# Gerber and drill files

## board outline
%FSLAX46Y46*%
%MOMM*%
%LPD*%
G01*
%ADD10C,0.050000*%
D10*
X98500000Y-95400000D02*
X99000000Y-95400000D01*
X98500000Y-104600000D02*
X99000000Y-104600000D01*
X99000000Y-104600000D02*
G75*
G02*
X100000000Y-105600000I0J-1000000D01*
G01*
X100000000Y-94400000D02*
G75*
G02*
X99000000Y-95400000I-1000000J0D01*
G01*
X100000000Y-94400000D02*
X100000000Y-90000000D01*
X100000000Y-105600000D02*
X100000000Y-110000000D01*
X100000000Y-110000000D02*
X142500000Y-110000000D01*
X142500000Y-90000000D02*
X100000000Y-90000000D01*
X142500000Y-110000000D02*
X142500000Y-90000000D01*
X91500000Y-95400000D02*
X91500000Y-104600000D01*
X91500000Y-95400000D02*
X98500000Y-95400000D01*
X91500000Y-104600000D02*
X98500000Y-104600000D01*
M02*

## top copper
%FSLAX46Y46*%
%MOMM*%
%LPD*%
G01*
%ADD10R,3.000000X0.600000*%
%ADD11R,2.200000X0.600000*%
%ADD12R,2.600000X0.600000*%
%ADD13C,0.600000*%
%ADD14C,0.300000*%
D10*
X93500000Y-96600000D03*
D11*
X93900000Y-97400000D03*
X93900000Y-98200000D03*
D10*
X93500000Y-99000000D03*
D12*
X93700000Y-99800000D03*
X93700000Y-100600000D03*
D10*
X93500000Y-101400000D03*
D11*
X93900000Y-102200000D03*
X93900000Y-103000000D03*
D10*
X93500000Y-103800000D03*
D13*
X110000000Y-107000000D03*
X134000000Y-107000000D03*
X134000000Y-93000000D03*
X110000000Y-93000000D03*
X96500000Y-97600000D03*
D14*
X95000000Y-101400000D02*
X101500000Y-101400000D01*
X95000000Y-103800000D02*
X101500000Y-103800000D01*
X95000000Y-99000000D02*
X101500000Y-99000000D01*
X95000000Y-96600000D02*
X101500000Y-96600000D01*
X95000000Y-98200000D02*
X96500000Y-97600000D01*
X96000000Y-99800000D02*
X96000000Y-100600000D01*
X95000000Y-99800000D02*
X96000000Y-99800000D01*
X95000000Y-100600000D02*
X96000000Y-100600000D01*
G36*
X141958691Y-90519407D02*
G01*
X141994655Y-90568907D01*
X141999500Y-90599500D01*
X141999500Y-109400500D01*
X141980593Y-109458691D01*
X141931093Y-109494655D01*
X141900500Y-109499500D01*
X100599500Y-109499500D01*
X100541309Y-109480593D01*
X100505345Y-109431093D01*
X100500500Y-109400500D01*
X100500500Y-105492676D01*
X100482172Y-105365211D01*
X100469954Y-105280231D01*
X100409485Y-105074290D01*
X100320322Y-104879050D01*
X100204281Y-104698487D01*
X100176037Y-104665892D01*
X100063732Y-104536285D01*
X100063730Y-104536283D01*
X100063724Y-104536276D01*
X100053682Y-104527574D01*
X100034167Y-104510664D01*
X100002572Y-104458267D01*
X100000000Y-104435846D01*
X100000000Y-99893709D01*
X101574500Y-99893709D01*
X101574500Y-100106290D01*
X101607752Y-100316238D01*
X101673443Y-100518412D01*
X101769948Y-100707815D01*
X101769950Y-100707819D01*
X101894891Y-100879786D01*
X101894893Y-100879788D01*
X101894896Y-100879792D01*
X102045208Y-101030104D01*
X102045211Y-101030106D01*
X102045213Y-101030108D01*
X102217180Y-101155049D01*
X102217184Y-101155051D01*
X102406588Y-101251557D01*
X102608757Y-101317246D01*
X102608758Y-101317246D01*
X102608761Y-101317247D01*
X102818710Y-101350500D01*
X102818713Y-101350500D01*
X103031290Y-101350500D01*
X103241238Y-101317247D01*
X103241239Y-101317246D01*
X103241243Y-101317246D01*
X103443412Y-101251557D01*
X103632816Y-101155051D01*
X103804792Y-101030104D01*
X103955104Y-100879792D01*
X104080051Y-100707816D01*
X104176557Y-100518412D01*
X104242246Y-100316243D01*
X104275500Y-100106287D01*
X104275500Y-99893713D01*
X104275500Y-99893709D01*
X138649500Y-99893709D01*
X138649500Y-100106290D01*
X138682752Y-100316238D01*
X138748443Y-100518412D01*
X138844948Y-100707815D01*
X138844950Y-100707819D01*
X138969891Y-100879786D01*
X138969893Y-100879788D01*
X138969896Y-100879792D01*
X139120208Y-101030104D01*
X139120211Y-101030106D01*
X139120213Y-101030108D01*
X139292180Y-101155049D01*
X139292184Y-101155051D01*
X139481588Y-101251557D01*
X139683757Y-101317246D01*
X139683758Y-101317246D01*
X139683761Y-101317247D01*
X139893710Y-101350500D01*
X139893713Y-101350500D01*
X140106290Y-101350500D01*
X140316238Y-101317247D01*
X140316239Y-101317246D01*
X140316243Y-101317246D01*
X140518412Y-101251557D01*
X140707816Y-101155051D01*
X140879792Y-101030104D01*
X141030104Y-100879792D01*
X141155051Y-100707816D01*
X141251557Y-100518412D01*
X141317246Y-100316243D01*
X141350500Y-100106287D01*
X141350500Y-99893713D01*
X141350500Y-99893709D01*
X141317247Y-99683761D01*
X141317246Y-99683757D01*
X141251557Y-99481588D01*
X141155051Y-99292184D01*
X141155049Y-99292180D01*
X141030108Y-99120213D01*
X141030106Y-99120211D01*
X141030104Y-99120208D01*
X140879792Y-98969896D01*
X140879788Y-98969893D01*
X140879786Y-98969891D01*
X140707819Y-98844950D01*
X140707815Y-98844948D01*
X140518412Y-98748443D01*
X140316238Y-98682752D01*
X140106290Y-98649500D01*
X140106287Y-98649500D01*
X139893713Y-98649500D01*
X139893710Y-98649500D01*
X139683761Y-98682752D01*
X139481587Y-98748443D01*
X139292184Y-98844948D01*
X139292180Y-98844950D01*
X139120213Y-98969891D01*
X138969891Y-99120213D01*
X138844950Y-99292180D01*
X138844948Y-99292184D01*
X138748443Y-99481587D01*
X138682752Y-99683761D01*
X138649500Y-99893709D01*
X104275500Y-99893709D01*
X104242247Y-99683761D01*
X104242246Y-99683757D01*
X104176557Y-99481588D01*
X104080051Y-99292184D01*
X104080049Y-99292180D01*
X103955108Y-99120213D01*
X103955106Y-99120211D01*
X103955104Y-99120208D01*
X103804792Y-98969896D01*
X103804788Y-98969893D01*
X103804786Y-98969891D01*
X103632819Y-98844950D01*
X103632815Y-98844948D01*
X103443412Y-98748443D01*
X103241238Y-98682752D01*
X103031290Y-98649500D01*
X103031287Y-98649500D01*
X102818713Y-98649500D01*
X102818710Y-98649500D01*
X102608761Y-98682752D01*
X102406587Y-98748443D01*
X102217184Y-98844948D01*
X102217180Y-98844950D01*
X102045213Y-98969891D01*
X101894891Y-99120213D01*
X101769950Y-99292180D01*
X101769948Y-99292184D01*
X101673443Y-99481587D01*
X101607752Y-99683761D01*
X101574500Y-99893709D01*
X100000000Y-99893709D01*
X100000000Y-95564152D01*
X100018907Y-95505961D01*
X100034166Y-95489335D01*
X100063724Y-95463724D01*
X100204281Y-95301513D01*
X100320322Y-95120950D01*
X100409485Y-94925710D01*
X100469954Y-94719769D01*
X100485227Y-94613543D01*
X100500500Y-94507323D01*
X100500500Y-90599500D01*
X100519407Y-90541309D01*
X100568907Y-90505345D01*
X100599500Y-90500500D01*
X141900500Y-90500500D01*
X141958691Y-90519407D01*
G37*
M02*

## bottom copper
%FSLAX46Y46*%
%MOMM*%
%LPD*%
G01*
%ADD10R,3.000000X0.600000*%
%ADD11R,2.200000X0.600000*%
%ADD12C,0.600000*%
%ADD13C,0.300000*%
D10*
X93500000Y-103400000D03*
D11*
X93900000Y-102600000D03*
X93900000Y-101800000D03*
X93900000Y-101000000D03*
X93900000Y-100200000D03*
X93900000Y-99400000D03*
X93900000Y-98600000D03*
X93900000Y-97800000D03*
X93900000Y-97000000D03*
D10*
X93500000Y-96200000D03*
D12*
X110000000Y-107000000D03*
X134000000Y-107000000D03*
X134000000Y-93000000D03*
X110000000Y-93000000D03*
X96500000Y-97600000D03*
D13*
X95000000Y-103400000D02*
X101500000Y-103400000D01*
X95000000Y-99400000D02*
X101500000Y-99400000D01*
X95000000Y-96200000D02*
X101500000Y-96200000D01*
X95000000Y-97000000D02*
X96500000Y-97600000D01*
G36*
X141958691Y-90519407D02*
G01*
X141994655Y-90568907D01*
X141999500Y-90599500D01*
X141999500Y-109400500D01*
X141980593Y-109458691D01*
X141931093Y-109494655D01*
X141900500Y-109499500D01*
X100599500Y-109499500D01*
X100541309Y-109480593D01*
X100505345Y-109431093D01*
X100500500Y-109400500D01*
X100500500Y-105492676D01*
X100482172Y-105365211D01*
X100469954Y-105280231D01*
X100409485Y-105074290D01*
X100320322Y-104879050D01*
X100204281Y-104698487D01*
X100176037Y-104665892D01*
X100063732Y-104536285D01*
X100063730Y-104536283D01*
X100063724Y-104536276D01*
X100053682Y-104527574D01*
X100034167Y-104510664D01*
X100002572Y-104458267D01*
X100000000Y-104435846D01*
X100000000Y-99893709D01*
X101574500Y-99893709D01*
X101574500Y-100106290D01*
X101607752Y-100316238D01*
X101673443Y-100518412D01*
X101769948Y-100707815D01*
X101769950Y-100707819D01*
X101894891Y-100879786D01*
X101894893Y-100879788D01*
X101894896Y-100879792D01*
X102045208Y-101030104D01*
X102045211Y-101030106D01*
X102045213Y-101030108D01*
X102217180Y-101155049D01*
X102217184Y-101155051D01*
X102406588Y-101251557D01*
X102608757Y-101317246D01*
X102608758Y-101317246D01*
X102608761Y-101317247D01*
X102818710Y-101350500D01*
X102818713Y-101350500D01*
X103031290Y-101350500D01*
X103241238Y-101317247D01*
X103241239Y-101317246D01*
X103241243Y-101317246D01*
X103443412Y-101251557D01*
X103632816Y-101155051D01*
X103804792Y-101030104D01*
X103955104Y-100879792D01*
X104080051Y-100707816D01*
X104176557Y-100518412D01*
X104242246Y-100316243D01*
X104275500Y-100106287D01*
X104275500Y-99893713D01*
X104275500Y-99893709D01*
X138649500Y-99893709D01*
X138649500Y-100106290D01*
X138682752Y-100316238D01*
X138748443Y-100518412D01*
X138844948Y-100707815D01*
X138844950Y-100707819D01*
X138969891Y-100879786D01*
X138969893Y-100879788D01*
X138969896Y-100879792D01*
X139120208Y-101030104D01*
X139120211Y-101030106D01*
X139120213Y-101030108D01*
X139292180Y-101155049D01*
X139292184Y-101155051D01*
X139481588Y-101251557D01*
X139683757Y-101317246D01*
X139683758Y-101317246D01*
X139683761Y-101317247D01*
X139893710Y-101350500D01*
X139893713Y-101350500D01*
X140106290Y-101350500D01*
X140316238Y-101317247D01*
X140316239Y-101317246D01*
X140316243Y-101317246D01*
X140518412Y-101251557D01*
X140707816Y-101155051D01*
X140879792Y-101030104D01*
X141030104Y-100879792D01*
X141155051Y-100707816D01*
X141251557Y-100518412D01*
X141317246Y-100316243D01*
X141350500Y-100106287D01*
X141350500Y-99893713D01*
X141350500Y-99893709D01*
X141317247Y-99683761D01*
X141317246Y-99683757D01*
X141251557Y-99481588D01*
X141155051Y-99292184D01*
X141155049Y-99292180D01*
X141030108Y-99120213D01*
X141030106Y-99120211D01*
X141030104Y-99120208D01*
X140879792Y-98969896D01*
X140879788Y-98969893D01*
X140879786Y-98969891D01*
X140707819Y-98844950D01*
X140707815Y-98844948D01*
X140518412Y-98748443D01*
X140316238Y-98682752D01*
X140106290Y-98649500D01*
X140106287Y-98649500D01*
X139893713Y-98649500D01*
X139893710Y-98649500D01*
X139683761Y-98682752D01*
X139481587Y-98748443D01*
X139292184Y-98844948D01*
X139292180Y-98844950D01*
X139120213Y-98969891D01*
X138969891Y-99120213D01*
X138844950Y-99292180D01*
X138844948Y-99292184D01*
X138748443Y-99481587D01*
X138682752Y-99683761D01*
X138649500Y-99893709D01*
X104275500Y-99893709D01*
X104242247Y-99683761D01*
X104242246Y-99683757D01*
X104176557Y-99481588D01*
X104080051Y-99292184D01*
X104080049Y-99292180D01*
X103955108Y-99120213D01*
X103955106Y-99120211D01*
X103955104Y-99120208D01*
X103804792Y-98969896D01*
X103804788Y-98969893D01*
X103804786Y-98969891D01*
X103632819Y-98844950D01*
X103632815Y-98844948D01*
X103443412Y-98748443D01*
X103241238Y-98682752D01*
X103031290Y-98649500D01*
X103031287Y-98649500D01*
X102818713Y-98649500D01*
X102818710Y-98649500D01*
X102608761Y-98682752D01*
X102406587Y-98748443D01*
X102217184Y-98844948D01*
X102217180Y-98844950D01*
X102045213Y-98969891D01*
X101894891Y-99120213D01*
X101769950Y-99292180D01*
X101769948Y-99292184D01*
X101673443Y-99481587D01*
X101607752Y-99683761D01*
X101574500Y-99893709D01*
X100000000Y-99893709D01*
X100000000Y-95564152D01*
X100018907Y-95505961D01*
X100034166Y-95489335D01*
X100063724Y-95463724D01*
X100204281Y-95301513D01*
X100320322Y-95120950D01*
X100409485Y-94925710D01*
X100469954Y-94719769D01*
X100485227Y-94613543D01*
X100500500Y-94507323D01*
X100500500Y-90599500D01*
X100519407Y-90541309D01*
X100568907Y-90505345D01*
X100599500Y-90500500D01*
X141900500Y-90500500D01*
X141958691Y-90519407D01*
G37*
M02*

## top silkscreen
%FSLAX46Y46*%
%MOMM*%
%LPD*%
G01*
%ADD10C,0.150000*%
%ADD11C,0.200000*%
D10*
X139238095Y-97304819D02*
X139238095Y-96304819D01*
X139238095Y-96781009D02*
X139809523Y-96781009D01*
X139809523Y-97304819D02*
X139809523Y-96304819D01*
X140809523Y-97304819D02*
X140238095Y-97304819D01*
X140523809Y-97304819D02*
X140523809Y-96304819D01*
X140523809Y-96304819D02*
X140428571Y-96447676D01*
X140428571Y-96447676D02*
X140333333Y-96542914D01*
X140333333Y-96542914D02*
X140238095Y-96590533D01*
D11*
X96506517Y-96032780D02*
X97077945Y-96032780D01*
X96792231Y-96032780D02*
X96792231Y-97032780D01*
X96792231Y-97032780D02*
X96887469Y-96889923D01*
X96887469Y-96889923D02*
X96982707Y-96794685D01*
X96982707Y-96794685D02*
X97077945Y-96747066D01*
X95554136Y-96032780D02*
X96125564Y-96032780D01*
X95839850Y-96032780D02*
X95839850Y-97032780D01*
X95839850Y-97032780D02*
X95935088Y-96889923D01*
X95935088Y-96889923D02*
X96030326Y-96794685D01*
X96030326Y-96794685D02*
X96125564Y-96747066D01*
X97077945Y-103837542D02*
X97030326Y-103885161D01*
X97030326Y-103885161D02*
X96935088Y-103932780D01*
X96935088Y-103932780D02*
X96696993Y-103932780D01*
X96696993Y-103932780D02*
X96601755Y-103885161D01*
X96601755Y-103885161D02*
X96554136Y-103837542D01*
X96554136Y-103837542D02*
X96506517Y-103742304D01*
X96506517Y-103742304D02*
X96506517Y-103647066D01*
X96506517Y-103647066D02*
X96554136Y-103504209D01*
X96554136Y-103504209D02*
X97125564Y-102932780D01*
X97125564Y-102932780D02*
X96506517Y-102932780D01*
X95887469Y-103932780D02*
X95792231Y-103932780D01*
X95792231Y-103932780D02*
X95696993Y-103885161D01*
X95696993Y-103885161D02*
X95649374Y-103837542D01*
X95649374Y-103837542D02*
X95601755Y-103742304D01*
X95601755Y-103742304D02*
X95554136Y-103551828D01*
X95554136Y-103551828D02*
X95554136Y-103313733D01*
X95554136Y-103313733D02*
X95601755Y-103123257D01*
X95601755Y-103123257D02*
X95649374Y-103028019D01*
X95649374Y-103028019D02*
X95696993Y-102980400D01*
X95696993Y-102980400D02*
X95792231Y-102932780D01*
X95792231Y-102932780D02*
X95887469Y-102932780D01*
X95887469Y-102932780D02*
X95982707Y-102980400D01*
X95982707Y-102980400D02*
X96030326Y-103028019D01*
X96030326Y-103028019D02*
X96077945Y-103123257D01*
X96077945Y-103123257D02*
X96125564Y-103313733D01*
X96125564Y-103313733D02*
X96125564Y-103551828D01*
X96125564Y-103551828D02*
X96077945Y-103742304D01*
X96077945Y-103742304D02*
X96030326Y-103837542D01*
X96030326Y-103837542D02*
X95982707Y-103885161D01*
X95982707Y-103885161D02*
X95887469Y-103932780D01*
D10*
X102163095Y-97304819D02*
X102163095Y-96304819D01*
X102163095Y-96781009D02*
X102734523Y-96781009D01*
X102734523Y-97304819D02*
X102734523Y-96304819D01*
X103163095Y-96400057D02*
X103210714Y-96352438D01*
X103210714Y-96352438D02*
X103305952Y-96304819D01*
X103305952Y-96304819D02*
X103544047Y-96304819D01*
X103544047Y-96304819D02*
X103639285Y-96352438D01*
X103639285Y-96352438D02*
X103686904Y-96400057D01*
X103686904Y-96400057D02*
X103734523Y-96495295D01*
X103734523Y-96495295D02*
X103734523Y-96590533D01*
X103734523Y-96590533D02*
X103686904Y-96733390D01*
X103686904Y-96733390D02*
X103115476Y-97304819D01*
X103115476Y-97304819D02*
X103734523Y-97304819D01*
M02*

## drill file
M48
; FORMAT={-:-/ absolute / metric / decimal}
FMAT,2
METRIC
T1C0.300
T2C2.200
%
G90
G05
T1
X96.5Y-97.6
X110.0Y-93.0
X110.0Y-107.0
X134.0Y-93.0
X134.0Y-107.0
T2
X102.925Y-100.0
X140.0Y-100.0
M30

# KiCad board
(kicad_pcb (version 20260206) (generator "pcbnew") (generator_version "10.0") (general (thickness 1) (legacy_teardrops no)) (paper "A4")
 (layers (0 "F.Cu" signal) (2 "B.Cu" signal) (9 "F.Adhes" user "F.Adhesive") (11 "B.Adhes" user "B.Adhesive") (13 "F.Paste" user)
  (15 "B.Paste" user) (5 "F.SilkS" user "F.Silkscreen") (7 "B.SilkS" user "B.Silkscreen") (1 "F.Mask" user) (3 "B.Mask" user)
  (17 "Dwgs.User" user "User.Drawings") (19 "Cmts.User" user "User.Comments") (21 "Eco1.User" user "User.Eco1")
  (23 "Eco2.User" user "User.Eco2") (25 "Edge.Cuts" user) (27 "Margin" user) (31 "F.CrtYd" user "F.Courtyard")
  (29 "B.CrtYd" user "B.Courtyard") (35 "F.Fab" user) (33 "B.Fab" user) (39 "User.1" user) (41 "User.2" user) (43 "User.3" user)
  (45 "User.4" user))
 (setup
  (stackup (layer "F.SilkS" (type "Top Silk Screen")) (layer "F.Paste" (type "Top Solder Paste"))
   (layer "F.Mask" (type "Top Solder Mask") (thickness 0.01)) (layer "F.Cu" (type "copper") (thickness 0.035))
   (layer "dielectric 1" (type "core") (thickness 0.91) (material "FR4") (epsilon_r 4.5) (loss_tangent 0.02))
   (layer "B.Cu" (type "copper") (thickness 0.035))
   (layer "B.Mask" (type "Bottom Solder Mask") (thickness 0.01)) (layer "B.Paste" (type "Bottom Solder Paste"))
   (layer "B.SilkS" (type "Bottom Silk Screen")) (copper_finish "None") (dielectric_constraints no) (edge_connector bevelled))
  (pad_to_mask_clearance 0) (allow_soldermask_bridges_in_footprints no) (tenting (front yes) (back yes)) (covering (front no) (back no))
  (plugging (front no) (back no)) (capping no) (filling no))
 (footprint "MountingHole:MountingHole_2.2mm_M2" (layer "F.Cu") (at 140 100)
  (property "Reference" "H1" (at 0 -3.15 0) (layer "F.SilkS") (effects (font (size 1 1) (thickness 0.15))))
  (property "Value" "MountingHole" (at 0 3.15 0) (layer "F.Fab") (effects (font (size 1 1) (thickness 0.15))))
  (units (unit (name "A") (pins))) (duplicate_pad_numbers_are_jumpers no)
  (pad "" np_thru_hole circle (at 0 0) (size 2.2 2.2) (drill 2.2) (layers "*.Cu" "*.Mask")))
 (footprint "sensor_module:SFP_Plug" (layer "F.Cu") (at 95 100 180)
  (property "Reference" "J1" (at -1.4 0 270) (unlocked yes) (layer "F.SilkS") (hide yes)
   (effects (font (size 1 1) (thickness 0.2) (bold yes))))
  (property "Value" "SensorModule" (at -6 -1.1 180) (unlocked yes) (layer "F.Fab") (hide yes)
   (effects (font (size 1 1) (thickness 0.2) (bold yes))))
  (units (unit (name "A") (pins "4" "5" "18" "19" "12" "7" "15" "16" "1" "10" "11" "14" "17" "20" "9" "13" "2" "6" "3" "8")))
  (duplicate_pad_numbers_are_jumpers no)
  (fp_line (start 3.5 4.6) (end 3.5 -4.6) (stroke (width 0.05) (type default)) (layer "Edge.Cuts"))
  (fp_line (start 3.5 4.6) (end -3.5 4.6) (stroke (width 0.05) (type solid)) (layer "Edge.Cuts"))
  (fp_line (start 3.5 -4.6) (end -3.5 -4.6) (stroke (width 0.05) (type solid)) (layer "Edge.Cuts"))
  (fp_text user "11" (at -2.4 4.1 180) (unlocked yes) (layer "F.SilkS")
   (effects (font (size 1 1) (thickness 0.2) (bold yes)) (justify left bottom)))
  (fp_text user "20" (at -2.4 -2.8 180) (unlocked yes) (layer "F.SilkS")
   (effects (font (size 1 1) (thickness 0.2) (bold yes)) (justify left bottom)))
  (pad "1" smd rect (at 1.5 -3.4 180) (size 3 0.6) (layers "B.Cu" "B.Mask") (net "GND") (thermal_bridge_angle 45))
  (pad "2" smd rect (at 1.1 -2.6 180) (size 2.2 0.6) (layers "B.Cu" "B.Mask") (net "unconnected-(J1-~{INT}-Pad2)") (thermal_bridge_angle 45))
  (pad "3" smd rect (at 1.1 -1.8 180) (size 2.2 0.6) (layers "B.Cu" "B.Mask") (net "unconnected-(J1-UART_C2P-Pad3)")
   (thermal_bridge_angle 45))
  (pad "4" smd rect (at 1.1 -1 180) (size 2.2 0.6) (layers "B.Cu" "B.Mask") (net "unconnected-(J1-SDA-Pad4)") (thermal_bridge_angle 45))
  (pad "5" smd rect (at 1.1 -0.2 180) (size 2.2 0.6) (layers "B.Cu" "B.Mask") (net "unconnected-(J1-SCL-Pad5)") (thermal_bridge_angle 45))
  (pad "6" smd rect (at 1.1 0.6 180) (size 2.2 0.6) (layers "B.Cu" "B.Mask") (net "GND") (thermal_bridge_angle 45))
  (pad "7" smd rect (at 1.1 1.4 180) (size 2.2 0.6) (layers "B.Cu" "B.Mask") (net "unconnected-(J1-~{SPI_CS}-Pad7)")
   (thermal_bridge_angle 45))
  (pad "8" smd rect (at 1.1 2.2 180) (size 2.2 0.6) (layers "B.Cu" "B.Mask") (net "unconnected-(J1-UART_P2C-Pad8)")
   (thermal_bridge_angle 45))
  (pad "9" smd rect (at 1.1 3 180) (size 2.2 0.6) (layers "B.Cu" "B.Mask") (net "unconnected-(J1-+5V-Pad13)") (thermal_bridge_angle 45))
  (pad "10" smd rect (at 1.5 3.8 180) (size 3 0.6) (layers "B.Cu" "B.Mask") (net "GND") (thermal_bridge_angle 45))
  (pad "11" smd rect (at 1.5 3.4 180) (size 3 0.6) (layers "F.Cu" "F.Mask") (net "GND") (thermal_bridge_angle 45))
  (pad "12" smd rect (at 1.1 2.6 180) (size 2.2 0.6) (layers "F.Cu" "F.Mask") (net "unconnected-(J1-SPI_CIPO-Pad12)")
   (thermal_bridge_angle 45))
  (pad "13" smd rect (at 1.1 1.8 180) (size 2.2 0.6) (layers "F.Cu" "F.Mask") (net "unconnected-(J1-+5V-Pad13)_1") (thermal_bridge_angle 45))
  (pad "14" smd rect (at 1.5 1 180) (size 3 0.6) (layers "F.Cu" "F.Mask") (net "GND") (thermal_bridge_angle 45))
  (pad "15" smd rect (at 1.3 0.2 180) (size 2.6 0.6) (layers "F.Cu" "F.Mask") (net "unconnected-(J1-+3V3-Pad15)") (thermal_bridge_angle 45))
  (pad "16" smd rect (at 1.3 -0.6 180) (size 2.6 0.6) (layers "F.Cu" "F.Mask") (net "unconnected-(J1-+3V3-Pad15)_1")
   (thermal_bridge_angle 45))
  (pad "17" smd rect (at 1.5 -1.4 180) (size 3 0.6) (layers "F.Cu" "F.Mask") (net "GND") (thermal_bridge_angle 45))
  (pad "18" smd rect (at 1.1 -2.2 180) (size 2.2 0.6) (layers "F.Cu" "F.Mask") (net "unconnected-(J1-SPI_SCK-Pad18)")
   (thermal_bridge_angle 45))
  (pad "19" smd rect (at 1.1 -3 180) (size 2.2 0.6) (layers "F.Cu" "F.Mask") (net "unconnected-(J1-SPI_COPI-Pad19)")
   (thermal_bridge_angle 45))
  (pad "20" smd rect (at 1.5 -3.8 180) (size 3 0.6) (layers "F.Cu" "F.Mask") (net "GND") (thermal_bridge_angle 45)))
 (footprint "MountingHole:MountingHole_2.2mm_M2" (layer "F.Cu") (at 102.925 100)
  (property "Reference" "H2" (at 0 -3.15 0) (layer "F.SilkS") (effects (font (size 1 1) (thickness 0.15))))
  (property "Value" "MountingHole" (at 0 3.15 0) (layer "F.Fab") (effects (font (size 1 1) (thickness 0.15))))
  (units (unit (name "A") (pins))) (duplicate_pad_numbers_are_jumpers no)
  (pad "" np_thru_hole circle (at 0 0) (size 2.2 2.2) (drill 2.2) (layers "*.Cu" "*.Mask")))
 (gr_line (start 98.5 95.4) (end 99 95.4) (stroke (width 0.05) (type default)) (layer "Edge.Cuts"))
 (gr_line (start 98.5 104.6) (end 99 104.6) (stroke (width 0.05) (type default)) (layer "Edge.Cuts"))
 (gr_arc (start 99 104.6) (mid 99.707107 104.892893) (end 100 105.6) (stroke (width 0.05) (type default)) (layer "Edge.Cuts"))
 (gr_arc (start 100 94.4) (mid 99.707107 95.107107) (end 99 95.4) (stroke (width 0.05) (type default)) (layer "Edge.Cuts"))
 (gr_line (start 100 94.4) (end 100 90) (stroke (width 0.05) (type default)) (layer "Edge.Cuts"))
 (gr_line (start 100 105.6) (end 100 110) (stroke (width 0.05) (type default)) (layer "Edge.Cuts"))
 (gr_line (start 100 110) (end 142.5 110) (stroke (width 0.05) (type default)) (layer "Edge.Cuts"))
 (gr_line (start 142.5 90) (end 100 90) (stroke (width 0.05) (type default)) (layer "Edge.Cuts"))
 (gr_line (start 142.5 110) (end 142.5 90) (stroke (width 0.05) (type default)) (layer "Edge.Cuts"))
 (segment (start 95 101.4) (end 101.5 101.4) (width 0.3) (layer "F.Cu") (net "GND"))
 (segment (start 95 103.8) (end 101.5 103.8) (width 0.3) (layer "F.Cu") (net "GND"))
 (segment (start 95 99) (end 101.5 99) (width 0.3) (layer "F.Cu") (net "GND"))
 (segment (start 95 96.6) (end 101.5 96.6) (width 0.3) (layer "F.Cu") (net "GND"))
 (via (at 110 107) (size 0.6) (drill 0.3) (layers "F.Cu" "B.Cu") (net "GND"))
 (via (at 134 107) (size 0.6) (drill 0.3) (layers "F.Cu" "B.Cu") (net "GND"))
 (via (at 134 93) (size 0.6) (drill 0.3) (layers "F.Cu" "B.Cu") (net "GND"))
 (via (at 110 93) (size 0.6) (drill 0.3) (layers "F.Cu" "B.Cu") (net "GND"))
 (segment (start 95 103.4) (end 101.5 103.4) (width 0.3) (layer "B.Cu") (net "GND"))
 (segment (start 95 99.4) (end 101.5 99.4) (width 0.3) (layer "B.Cu") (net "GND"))
 (segment (start 95 96.2) (end 101.5 96.2) (width 0.3) (layer "B.Cu") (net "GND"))
 (segment (start 95 98.2) (end 96.5 97.6) (width 0.3) (layer "F.Cu") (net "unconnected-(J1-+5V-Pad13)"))
 (via (at 96.5 97.6) (size 0.6) (drill 0.3) (layers "F.Cu" "B.Cu") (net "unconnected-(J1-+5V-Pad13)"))
 (segment (start 95 97) (end 96.5 97.6) (width 0.3) (layer "B.Cu") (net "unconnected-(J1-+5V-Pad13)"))
 (segment (start 96 99.8) (end 96 100.6) (width 0.3) (layer "F.Cu") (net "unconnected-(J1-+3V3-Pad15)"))
 (segment (start 95 99.8) (end 96 99.8) (width 0.3) (layer "F.Cu") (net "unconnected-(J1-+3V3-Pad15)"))
 (segment (start 95 100.6) (end 96 100.6) (width 0.3) (layer "F.Cu") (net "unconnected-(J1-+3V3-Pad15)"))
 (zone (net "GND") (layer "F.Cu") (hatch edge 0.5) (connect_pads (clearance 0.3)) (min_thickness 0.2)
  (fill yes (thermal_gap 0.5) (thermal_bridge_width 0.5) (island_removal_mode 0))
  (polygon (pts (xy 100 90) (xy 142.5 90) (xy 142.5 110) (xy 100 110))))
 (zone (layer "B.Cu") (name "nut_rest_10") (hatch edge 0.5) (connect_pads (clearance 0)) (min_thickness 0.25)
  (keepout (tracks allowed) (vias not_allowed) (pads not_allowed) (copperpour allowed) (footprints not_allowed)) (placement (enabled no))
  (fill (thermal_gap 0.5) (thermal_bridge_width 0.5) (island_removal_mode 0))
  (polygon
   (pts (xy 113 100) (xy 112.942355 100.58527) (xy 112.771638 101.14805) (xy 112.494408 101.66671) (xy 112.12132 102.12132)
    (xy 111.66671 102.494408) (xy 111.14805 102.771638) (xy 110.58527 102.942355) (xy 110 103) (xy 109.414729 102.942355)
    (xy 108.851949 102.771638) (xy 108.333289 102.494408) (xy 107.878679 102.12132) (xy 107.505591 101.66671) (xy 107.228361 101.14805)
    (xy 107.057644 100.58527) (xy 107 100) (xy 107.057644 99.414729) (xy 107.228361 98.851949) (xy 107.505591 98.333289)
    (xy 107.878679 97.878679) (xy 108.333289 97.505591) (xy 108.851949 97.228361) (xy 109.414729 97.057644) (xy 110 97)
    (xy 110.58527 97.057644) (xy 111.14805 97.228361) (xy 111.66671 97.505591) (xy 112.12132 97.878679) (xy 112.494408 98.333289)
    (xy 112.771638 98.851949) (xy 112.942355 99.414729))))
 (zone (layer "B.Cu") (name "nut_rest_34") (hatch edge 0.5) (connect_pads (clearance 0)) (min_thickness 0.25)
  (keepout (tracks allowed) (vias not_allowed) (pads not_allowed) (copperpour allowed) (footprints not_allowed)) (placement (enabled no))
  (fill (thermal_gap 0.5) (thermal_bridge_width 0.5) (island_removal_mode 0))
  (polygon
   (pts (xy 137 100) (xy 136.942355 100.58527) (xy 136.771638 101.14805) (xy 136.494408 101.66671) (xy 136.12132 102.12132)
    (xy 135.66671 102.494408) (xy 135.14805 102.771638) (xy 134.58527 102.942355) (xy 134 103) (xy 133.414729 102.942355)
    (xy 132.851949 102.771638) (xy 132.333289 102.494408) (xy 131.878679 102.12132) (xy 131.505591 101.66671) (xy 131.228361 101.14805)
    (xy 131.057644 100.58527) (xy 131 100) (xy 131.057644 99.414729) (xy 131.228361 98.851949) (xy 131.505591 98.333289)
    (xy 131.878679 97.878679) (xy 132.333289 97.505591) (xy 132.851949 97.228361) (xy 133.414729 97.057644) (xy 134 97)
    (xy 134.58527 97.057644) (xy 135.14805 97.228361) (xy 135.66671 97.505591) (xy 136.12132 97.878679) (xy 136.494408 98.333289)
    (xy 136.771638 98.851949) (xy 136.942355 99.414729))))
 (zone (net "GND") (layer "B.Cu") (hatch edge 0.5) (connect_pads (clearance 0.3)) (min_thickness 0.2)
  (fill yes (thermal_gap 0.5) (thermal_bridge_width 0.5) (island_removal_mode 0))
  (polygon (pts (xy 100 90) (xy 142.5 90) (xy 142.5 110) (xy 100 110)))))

